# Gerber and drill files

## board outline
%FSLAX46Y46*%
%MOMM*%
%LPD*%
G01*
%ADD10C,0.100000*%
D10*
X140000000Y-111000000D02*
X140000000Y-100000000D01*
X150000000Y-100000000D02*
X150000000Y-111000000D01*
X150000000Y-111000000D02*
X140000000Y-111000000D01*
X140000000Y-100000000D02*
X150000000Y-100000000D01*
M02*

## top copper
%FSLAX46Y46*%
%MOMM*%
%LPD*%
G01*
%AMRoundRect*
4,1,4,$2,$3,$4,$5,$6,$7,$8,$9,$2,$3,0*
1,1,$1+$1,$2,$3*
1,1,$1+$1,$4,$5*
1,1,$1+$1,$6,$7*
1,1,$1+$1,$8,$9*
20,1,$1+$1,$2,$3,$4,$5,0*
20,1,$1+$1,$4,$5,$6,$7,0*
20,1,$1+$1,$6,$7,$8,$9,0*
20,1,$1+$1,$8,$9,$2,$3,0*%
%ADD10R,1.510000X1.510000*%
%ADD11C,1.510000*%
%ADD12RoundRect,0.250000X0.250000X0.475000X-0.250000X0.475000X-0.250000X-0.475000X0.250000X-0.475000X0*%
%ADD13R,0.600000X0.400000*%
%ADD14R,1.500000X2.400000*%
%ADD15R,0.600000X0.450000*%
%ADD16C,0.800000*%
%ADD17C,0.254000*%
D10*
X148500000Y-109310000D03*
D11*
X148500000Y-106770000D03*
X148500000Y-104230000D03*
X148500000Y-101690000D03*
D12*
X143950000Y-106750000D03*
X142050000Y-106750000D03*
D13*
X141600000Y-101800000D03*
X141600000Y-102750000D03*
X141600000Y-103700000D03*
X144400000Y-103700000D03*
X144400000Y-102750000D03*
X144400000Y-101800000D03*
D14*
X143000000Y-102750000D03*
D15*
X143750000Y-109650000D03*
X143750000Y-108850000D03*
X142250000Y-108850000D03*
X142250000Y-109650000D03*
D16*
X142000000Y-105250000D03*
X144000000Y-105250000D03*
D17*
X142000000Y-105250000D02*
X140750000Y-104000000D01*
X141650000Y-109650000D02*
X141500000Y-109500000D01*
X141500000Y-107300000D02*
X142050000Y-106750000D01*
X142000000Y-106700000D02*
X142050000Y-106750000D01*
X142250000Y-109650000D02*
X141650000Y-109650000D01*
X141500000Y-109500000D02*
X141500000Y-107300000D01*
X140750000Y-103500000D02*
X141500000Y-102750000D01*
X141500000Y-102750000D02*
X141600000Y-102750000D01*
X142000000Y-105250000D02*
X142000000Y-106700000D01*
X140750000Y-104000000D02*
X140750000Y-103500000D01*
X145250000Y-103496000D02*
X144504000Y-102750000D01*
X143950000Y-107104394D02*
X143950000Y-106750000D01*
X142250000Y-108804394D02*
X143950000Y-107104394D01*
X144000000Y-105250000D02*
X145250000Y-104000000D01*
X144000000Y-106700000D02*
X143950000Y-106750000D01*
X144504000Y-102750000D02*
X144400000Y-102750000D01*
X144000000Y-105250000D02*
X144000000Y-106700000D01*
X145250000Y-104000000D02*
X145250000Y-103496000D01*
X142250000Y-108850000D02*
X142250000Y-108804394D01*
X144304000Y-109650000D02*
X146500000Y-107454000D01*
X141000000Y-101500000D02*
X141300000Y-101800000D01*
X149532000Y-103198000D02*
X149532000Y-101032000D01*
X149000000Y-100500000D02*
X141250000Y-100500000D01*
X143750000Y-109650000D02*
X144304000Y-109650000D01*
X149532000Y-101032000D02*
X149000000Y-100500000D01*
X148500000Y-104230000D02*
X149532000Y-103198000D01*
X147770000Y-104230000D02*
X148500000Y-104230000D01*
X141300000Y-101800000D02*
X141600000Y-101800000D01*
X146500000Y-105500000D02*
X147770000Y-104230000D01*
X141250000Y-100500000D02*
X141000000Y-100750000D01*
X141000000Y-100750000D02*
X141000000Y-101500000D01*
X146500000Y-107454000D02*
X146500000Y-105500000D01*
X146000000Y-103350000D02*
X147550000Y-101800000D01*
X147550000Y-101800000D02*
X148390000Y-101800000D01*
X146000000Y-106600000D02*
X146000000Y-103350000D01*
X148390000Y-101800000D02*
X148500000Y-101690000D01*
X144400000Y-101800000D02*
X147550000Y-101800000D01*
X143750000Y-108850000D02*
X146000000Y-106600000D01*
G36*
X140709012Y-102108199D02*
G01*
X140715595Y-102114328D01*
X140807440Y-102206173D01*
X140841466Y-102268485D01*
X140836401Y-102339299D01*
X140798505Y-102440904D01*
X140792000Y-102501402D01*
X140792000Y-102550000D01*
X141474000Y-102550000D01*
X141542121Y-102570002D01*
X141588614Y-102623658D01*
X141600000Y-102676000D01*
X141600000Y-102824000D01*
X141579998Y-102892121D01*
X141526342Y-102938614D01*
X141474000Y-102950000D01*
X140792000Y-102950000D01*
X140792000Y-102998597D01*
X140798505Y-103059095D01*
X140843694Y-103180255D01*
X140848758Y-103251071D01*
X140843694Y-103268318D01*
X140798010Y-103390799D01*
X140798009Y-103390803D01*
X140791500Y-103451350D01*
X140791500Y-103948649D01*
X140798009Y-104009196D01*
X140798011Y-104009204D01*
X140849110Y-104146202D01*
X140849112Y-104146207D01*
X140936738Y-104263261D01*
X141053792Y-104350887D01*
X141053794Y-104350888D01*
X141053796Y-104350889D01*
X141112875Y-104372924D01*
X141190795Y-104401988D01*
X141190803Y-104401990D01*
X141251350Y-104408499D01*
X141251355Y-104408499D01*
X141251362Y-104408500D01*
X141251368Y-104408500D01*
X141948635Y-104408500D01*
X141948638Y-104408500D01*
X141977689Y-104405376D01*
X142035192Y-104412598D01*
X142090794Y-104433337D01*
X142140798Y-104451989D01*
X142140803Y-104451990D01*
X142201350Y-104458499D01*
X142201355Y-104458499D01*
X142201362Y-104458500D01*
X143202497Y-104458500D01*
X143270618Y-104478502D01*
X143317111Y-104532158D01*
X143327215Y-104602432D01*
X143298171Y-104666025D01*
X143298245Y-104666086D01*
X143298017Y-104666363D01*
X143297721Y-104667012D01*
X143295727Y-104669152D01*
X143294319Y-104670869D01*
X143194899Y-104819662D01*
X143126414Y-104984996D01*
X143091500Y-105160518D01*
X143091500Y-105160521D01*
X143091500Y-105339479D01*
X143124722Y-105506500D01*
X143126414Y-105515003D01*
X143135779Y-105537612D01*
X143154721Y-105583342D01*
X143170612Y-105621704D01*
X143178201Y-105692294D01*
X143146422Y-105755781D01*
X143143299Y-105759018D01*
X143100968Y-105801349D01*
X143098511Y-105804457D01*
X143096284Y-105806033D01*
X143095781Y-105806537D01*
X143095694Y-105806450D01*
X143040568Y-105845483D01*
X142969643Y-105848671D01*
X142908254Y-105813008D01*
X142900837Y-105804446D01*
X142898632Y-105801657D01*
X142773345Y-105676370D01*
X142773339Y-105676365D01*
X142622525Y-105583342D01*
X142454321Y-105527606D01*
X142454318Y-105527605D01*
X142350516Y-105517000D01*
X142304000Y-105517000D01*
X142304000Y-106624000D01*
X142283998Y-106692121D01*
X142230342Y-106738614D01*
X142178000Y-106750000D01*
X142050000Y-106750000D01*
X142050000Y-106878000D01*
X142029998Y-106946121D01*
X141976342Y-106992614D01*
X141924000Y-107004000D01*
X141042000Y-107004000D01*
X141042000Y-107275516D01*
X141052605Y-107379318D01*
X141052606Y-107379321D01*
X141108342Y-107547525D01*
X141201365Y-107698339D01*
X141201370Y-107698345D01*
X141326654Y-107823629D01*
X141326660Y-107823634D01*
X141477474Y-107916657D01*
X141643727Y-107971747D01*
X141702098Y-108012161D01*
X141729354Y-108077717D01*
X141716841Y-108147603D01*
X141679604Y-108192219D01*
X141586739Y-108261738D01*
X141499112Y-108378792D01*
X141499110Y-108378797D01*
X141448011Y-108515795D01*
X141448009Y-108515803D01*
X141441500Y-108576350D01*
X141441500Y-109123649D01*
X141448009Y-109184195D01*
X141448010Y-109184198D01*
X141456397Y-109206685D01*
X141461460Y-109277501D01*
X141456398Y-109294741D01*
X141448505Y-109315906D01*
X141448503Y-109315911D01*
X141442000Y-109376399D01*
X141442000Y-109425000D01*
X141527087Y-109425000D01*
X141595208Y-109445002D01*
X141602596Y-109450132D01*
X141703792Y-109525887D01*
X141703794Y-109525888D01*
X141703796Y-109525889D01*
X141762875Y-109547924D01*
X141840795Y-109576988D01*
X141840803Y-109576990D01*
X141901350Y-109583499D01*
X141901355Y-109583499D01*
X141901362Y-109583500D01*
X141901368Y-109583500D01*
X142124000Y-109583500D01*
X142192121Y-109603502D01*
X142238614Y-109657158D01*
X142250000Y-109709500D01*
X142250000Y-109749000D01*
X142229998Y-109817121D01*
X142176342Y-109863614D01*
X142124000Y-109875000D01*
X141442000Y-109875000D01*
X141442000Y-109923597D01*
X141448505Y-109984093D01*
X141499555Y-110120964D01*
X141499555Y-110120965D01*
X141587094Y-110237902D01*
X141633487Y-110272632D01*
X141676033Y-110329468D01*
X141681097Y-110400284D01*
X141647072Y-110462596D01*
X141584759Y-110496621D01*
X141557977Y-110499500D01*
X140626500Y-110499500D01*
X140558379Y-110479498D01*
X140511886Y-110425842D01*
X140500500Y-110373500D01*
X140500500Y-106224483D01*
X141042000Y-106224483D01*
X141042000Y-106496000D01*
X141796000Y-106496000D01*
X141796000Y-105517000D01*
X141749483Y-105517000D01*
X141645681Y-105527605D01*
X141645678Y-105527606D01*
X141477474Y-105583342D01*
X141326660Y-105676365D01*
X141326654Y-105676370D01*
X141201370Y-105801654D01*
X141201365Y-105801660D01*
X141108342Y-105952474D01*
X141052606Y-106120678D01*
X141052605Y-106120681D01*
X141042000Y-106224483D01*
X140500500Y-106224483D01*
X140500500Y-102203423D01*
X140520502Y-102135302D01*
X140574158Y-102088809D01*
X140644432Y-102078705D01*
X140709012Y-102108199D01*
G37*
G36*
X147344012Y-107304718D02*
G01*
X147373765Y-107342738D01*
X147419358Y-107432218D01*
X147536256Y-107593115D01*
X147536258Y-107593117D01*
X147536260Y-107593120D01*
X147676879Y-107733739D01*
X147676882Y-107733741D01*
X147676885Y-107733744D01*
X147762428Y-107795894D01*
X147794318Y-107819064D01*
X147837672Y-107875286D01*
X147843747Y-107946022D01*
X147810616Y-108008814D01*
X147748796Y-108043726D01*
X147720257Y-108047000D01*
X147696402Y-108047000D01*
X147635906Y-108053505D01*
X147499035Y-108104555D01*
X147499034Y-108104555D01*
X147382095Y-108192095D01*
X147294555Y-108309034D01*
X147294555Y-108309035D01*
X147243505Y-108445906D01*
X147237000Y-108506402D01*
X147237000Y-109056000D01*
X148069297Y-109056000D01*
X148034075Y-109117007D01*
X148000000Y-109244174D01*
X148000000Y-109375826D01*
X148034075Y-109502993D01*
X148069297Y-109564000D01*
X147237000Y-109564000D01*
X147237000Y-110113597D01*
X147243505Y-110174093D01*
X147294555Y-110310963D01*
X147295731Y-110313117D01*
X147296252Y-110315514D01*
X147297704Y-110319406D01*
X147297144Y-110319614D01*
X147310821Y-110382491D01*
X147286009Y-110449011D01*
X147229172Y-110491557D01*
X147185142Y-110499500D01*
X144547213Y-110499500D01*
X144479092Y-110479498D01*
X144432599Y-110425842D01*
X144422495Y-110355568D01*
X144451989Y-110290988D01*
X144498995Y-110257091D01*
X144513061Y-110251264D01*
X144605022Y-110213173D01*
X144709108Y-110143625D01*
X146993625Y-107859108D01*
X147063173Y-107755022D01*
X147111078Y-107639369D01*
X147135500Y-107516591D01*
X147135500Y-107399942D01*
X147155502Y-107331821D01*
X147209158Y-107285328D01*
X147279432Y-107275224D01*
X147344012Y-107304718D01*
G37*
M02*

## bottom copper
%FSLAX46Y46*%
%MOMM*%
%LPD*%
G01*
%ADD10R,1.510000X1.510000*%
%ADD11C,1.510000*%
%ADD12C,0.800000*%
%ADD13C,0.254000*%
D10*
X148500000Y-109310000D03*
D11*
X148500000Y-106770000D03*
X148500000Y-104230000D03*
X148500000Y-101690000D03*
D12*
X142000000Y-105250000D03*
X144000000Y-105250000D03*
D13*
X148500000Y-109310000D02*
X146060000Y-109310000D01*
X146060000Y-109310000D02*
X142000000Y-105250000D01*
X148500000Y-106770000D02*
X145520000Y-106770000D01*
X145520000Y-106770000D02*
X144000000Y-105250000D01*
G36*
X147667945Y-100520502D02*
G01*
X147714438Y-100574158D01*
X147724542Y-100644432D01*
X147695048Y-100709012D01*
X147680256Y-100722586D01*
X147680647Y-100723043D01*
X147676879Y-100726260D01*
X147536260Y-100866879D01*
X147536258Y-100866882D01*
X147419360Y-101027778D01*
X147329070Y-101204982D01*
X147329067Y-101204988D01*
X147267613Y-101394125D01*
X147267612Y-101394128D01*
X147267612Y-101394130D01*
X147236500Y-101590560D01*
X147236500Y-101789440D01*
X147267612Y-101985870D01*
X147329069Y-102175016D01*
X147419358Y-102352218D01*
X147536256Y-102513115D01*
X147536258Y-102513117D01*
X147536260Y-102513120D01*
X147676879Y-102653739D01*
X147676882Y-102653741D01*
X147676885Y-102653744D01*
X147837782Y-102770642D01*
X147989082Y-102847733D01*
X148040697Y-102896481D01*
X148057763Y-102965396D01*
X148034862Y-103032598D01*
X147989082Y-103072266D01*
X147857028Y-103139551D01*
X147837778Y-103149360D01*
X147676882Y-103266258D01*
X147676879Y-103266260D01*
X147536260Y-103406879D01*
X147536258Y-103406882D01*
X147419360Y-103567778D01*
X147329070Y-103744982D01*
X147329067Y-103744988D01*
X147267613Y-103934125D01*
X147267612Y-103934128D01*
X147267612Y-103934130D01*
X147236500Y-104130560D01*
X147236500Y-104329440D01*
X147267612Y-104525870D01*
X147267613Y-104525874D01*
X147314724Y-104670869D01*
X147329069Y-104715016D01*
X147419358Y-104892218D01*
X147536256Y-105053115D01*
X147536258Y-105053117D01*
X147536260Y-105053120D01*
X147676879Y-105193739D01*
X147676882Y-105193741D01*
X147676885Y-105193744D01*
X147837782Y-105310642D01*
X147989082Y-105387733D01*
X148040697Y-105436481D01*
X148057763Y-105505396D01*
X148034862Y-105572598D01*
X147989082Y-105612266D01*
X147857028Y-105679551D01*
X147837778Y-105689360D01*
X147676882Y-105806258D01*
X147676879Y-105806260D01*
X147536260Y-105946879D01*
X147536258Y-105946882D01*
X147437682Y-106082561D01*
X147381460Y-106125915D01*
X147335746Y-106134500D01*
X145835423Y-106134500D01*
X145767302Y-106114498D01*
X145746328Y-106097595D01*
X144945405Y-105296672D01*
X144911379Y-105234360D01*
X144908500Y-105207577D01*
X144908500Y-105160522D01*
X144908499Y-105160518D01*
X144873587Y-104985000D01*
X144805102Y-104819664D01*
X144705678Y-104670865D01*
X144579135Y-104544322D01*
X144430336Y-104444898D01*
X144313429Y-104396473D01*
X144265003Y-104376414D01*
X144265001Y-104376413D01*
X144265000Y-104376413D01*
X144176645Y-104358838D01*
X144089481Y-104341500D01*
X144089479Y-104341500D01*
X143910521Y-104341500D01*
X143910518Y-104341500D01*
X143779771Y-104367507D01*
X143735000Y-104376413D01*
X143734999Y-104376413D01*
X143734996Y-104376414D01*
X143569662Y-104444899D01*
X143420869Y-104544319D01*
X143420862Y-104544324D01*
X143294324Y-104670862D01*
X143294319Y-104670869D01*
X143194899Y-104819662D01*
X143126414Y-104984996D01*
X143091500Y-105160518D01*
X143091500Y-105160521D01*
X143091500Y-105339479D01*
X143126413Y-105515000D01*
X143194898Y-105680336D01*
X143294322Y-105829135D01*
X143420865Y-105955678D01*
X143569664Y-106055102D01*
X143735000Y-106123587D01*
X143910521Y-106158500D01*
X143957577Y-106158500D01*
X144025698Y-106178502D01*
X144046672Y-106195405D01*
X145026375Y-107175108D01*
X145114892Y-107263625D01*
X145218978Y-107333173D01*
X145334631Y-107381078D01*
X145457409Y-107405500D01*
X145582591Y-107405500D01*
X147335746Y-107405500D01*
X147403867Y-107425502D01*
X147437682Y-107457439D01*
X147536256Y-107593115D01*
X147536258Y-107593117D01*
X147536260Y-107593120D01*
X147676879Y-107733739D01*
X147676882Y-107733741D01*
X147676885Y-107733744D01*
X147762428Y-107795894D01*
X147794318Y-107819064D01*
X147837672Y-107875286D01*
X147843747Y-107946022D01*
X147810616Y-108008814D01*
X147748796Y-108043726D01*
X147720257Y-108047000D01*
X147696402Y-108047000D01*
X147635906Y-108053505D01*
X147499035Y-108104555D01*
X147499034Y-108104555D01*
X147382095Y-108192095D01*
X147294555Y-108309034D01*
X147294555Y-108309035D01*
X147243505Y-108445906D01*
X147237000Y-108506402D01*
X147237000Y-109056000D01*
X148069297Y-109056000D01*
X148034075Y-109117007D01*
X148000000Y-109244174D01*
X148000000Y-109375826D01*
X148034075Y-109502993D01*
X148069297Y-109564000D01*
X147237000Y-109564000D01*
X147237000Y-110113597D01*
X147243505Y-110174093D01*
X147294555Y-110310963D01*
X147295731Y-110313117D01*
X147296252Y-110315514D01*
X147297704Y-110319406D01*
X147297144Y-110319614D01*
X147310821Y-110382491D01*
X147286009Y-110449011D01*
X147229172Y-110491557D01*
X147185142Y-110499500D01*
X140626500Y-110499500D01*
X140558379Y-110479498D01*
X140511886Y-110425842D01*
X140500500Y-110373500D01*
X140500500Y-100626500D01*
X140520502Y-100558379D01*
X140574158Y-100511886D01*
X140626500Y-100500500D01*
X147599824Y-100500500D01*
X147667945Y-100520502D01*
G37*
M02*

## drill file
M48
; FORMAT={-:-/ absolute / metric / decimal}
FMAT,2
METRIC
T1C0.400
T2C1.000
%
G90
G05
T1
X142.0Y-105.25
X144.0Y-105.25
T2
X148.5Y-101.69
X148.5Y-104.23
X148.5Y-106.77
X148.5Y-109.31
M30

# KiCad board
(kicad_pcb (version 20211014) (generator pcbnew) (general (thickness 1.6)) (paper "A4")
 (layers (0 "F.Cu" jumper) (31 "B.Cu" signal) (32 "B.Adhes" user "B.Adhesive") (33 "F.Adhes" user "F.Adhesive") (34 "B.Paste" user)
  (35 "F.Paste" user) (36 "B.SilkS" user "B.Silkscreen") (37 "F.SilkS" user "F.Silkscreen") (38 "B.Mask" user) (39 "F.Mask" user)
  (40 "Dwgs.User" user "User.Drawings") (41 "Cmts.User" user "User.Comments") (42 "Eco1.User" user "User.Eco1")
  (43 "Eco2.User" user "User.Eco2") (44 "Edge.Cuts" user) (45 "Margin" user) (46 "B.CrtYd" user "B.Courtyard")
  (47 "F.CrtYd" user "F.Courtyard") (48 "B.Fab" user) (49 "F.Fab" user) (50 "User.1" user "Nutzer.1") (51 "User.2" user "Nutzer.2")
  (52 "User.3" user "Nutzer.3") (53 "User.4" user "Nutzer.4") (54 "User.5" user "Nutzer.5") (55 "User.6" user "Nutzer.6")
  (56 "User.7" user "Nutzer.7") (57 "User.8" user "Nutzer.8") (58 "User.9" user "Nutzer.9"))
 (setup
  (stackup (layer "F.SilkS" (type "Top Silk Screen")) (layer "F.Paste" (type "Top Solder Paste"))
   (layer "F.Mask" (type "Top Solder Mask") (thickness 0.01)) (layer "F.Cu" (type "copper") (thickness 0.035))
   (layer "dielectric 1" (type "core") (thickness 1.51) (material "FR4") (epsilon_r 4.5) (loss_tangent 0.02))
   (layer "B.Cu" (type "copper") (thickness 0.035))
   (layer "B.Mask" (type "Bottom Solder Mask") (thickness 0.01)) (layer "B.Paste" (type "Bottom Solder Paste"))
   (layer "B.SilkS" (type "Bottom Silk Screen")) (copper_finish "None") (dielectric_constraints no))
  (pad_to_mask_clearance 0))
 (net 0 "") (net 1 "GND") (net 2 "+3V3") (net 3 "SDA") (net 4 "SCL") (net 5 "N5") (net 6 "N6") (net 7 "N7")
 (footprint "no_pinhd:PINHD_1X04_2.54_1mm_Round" (layer "F.Cu") (at 148.5 105.5 90) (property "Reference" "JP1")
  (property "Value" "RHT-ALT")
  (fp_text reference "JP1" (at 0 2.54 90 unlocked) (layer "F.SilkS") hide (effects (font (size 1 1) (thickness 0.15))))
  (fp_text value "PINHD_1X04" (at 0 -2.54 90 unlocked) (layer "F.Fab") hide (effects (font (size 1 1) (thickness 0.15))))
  (pad "1" thru_hole rect (at -3.81 0 90) (size 1.51 1.51) (drill 1) (layers *.Cu *.Mask) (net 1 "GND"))
  (pad "2" thru_hole circle (at -1.27 0 90) (size 1.51 1.51) (drill 1) (layers *.Cu *.Mask) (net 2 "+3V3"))
  (pad "3" thru_hole circle (at 1.27 0 90) (size 1.51 1.51) (drill 1) (layers *.Cu *.Mask) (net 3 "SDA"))
  (pad "4" thru_hole circle (at 3.81 0 90) (size 1.51 1.51) (drill 1) (layers *.Cu *.Mask) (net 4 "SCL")))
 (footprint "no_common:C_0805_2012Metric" (layer "F.Cu") (at 143 106.75 180) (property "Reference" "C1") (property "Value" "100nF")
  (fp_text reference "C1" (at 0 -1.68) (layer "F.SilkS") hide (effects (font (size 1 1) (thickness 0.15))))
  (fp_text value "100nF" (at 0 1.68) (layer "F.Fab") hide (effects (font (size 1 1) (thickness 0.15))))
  (pad "1" smd roundrect (at -0.95 0 180) (size 1 1.45) (layers "F.Cu" "F.Mask") (roundrect_rratio 0.25) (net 2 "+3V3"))
  (pad "2" smd roundrect (at 0.95 0 180) (size 1 1.45) (layers "F.Cu" "F.Mask") (roundrect_rratio 0.25) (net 1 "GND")))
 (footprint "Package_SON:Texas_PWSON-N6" (layer "F.Cu") (at 143 102.75)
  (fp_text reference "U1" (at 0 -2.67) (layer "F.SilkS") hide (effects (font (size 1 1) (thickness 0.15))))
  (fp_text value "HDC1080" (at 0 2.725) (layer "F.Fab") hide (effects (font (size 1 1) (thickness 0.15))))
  (pad "1" smd rect (at -1.4 -0.95) (size 0.6 0.4) (layers "F.Cu" "F.Paste" "F.Mask") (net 3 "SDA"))
  (pad "2" smd rect (at -1.4 0) (size 0.6 0.4) (layers "F.Cu" "F.Paste" "F.Mask") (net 1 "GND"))
  (pad "3" smd rect (at -1.4 0.95) (size 0.6 0.4) (layers "F.Cu" "F.Paste" "F.Mask") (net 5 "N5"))
  (pad "4" smd rect (at 1.4 0.95) (size 0.6 0.4) (layers "F.Cu" "F.Paste" "F.Mask") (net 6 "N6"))
  (pad "5" smd rect (at 1.4 0) (size 0.6 0.4) (layers "F.Cu" "F.Paste" "F.Mask") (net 2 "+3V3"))
  (pad "6" smd rect (at 1.4 -0.95) (size 0.6 0.4) (layers "F.Cu" "F.Paste" "F.Mask") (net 4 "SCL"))
  (pad "7" smd rect (at 0 0) (size 1.5 2.4) (layers "F.Cu" "F.Paste" "F.Mask") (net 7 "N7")))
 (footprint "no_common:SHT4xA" (layer "F.Cu") (at 143 109.25 180)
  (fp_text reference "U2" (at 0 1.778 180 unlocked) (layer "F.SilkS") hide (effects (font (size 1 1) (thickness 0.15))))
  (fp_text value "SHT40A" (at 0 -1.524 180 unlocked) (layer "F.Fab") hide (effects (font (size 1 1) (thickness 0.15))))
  (pad "1" smd rect (at -0.75 -0.4 180) (size 0.6 0.45) (layers "F.Cu" "F.Paste" "F.Mask") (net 3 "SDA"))
  (pad "2" smd rect (at -0.75 0.4 180) (size 0.6 0.45) (layers "F.Cu" "F.Paste" "F.Mask") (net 4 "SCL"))
  (pad "3" smd rect (at 0.75 0.4 180) (size 0.6 0.45) (layers "F.Cu" "F.Paste" "F.Mask") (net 2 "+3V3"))
  (pad "4" smd rect (at 0.75 -0.4 180) (size 0.6 0.45) (layers "F.Cu" "F.Paste" "F.Mask") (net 1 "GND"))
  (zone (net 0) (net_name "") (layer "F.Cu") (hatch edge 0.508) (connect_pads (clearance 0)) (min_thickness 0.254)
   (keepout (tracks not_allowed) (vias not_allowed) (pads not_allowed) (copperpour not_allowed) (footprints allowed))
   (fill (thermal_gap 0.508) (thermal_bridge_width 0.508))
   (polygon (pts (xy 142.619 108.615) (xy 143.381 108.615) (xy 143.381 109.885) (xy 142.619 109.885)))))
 (gr_line (start 140 111) (end 140 100) (layer "Edge.Cuts") (width 0.1))
 (gr_line (start 150 100) (end 150 111) (layer "Edge.Cuts") (width 0.1))
 (gr_line (start 150 111) (end 140 111) (layer "Edge.Cuts") (width 0.1))
 (gr_line (start 140 100) (end 150 100) (layer "Edge.Cuts") (width 0.1))
 (segment (start 142 105.25) (end 140.75 104) (width 0.254) (layer "F.Cu") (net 1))
 (segment (start 141.65 109.65) (end 141.5 109.5) (width 0.254) (layer "F.Cu") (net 1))
 (segment (start 141.5 107.3) (end 142.05 106.75) (width 0.254) (layer "F.Cu") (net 1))
 (segment (start 142 106.7) (end 142.05 106.75) (width 0.254) (layer "F.Cu") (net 1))
 (segment (start 142.25 109.65) (end 141.65 109.65) (width 0.254) (layer "F.Cu") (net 1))
 (segment (start 141.5 109.5) (end 141.5 107.3) (width 0.254) (layer "F.Cu") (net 1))
 (segment (start 140.75 103.5) (end 141.5 102.75) (width 0.254) (layer "F.Cu") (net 1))
 (segment (start 141.5 102.75) (end 141.6 102.75) (width 0.254) (layer "F.Cu") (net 1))
 (segment (start 142 105.25) (end 142 106.7) (width 0.254) (layer "F.Cu") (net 1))
 (segment (start 140.75 104) (end 140.75 103.5) (width 0.254) (layer "F.Cu") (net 1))
 (via (at 142 105.25) (size 0.8) (drill 0.4) (layers "F.Cu" "B.Cu") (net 1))
 (segment (start 148.5 109.31) (end 146.06 109.31) (width 0.254) (layer "B.Cu") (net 1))
 (segment (start 146.06 109.31) (end 142 105.25) (width 0.254) (layer "B.Cu") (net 1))
 (segment (start 145.25 103.496) (end 144.504 102.75) (width 0.254) (layer "F.Cu") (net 2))
 (segment (start 143.95 107.104394) (end 143.95 106.75) (width 0.254) (layer "F.Cu") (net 2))
 (segment (start 142.25 108.804394) (end 143.95 107.104394) (width 0.254) (layer "F.Cu") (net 2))
 (segment (start 144 105.25) (end 145.25 104) (width 0.254) (layer "F.Cu") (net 2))
 (segment (start 144 106.7) (end 143.95 106.75) (width 0.254) (layer "F.Cu") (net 2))
 (segment (start 144.504 102.75) (end 144.4 102.75) (width 0.254) (layer "F.Cu") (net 2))
 (segment (start 144 105.25) (end 144 106.7) (width 0.254) (layer "F.Cu") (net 2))
 (segment (start 145.25 104) (end 145.25 103.496) (width 0.254) (layer "F.Cu") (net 2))
 (segment (start 142.25 108.85) (end 142.25 108.804394) (width 0.254) (layer "F.Cu") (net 2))
 (via (at 144 105.25) (size 0.8) (drill 0.4) (layers "F.Cu" "B.Cu") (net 2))
 (segment (start 148.5 106.77) (end 145.52 106.77) (width 0.254) (layer "B.Cu") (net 2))
 (segment (start 145.52 106.77) (end 144 105.25) (width 0.254) (layer "B.Cu") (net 2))
 (segment (start 144.304 109.65) (end 146.5 107.454) (width 0.254) (layer "F.Cu") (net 3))
 (segment (start 141 101.5) (end 141.3 101.8) (width 0.254) (layer "F.Cu") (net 3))
 (segment (start 149.532 103.198) (end 149.532 101.032) (width 0.254) (layer "F.Cu") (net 3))
 (segment (start 149 100.5) (end 141.25 100.5) (width 0.254) (layer "F.Cu") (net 3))
 (segment (start 143.75 109.65) (end 144.304 109.65) (width 0.254) (layer "F.Cu") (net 3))
 (segment (start 149.532 101.032) (end 149 100.5) (width 0.254) (layer "F.Cu") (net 3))
 (segment (start 148.5 104.23) (end 149.532 103.198) (width 0.254) (layer "F.Cu") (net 3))
 (segment (start 147.77 104.23) (end 148.5 104.23) (width 0.254) (layer "F.Cu") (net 3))
 (segment (start 141.3 101.8) (end 141.6 101.8) (width 0.254) (layer "F.Cu") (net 3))
 (segment (start 146.5 105.5) (end 147.77 104.23) (width 0.254) (layer "F.Cu") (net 3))
 (segment (start 141.25 100.5) (end 141 100.75) (width 0.254) (layer "F.Cu") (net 3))
 (segment (start 141 100.75) (end 141 101.5) (width 0.254) (layer "F.Cu") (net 3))
 (segment (start 146.5 107.454) (end 146.5 105.5) (width 0.254) (layer "F.Cu") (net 3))
 (segment (start 146 103.35) (end 147.55 101.8) (width 0.254) (layer "F.Cu") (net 4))
 (segment (start 147.55 101.8) (end 148.39 101.8) (width 0.254) (layer "F.Cu") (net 4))
 (segment (start 146 106.6) (end 146 103.35) (width 0.254) (layer "F.Cu") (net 4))
 (segment (start 148.39 101.8) (end 148.5 101.69) (width 0.254) (layer "F.Cu") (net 4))
 (segment (start 144.4 101.8) (end 147.55 101.8) (width 0.254) (layer "F.Cu") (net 4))
 (segment (start 143.75 108.85) (end 146 106.6) (width 0.254) (layer "F.Cu") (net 4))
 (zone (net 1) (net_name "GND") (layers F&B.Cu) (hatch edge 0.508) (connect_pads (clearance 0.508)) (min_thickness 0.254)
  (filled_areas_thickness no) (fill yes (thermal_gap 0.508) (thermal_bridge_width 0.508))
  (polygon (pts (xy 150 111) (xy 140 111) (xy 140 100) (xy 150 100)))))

